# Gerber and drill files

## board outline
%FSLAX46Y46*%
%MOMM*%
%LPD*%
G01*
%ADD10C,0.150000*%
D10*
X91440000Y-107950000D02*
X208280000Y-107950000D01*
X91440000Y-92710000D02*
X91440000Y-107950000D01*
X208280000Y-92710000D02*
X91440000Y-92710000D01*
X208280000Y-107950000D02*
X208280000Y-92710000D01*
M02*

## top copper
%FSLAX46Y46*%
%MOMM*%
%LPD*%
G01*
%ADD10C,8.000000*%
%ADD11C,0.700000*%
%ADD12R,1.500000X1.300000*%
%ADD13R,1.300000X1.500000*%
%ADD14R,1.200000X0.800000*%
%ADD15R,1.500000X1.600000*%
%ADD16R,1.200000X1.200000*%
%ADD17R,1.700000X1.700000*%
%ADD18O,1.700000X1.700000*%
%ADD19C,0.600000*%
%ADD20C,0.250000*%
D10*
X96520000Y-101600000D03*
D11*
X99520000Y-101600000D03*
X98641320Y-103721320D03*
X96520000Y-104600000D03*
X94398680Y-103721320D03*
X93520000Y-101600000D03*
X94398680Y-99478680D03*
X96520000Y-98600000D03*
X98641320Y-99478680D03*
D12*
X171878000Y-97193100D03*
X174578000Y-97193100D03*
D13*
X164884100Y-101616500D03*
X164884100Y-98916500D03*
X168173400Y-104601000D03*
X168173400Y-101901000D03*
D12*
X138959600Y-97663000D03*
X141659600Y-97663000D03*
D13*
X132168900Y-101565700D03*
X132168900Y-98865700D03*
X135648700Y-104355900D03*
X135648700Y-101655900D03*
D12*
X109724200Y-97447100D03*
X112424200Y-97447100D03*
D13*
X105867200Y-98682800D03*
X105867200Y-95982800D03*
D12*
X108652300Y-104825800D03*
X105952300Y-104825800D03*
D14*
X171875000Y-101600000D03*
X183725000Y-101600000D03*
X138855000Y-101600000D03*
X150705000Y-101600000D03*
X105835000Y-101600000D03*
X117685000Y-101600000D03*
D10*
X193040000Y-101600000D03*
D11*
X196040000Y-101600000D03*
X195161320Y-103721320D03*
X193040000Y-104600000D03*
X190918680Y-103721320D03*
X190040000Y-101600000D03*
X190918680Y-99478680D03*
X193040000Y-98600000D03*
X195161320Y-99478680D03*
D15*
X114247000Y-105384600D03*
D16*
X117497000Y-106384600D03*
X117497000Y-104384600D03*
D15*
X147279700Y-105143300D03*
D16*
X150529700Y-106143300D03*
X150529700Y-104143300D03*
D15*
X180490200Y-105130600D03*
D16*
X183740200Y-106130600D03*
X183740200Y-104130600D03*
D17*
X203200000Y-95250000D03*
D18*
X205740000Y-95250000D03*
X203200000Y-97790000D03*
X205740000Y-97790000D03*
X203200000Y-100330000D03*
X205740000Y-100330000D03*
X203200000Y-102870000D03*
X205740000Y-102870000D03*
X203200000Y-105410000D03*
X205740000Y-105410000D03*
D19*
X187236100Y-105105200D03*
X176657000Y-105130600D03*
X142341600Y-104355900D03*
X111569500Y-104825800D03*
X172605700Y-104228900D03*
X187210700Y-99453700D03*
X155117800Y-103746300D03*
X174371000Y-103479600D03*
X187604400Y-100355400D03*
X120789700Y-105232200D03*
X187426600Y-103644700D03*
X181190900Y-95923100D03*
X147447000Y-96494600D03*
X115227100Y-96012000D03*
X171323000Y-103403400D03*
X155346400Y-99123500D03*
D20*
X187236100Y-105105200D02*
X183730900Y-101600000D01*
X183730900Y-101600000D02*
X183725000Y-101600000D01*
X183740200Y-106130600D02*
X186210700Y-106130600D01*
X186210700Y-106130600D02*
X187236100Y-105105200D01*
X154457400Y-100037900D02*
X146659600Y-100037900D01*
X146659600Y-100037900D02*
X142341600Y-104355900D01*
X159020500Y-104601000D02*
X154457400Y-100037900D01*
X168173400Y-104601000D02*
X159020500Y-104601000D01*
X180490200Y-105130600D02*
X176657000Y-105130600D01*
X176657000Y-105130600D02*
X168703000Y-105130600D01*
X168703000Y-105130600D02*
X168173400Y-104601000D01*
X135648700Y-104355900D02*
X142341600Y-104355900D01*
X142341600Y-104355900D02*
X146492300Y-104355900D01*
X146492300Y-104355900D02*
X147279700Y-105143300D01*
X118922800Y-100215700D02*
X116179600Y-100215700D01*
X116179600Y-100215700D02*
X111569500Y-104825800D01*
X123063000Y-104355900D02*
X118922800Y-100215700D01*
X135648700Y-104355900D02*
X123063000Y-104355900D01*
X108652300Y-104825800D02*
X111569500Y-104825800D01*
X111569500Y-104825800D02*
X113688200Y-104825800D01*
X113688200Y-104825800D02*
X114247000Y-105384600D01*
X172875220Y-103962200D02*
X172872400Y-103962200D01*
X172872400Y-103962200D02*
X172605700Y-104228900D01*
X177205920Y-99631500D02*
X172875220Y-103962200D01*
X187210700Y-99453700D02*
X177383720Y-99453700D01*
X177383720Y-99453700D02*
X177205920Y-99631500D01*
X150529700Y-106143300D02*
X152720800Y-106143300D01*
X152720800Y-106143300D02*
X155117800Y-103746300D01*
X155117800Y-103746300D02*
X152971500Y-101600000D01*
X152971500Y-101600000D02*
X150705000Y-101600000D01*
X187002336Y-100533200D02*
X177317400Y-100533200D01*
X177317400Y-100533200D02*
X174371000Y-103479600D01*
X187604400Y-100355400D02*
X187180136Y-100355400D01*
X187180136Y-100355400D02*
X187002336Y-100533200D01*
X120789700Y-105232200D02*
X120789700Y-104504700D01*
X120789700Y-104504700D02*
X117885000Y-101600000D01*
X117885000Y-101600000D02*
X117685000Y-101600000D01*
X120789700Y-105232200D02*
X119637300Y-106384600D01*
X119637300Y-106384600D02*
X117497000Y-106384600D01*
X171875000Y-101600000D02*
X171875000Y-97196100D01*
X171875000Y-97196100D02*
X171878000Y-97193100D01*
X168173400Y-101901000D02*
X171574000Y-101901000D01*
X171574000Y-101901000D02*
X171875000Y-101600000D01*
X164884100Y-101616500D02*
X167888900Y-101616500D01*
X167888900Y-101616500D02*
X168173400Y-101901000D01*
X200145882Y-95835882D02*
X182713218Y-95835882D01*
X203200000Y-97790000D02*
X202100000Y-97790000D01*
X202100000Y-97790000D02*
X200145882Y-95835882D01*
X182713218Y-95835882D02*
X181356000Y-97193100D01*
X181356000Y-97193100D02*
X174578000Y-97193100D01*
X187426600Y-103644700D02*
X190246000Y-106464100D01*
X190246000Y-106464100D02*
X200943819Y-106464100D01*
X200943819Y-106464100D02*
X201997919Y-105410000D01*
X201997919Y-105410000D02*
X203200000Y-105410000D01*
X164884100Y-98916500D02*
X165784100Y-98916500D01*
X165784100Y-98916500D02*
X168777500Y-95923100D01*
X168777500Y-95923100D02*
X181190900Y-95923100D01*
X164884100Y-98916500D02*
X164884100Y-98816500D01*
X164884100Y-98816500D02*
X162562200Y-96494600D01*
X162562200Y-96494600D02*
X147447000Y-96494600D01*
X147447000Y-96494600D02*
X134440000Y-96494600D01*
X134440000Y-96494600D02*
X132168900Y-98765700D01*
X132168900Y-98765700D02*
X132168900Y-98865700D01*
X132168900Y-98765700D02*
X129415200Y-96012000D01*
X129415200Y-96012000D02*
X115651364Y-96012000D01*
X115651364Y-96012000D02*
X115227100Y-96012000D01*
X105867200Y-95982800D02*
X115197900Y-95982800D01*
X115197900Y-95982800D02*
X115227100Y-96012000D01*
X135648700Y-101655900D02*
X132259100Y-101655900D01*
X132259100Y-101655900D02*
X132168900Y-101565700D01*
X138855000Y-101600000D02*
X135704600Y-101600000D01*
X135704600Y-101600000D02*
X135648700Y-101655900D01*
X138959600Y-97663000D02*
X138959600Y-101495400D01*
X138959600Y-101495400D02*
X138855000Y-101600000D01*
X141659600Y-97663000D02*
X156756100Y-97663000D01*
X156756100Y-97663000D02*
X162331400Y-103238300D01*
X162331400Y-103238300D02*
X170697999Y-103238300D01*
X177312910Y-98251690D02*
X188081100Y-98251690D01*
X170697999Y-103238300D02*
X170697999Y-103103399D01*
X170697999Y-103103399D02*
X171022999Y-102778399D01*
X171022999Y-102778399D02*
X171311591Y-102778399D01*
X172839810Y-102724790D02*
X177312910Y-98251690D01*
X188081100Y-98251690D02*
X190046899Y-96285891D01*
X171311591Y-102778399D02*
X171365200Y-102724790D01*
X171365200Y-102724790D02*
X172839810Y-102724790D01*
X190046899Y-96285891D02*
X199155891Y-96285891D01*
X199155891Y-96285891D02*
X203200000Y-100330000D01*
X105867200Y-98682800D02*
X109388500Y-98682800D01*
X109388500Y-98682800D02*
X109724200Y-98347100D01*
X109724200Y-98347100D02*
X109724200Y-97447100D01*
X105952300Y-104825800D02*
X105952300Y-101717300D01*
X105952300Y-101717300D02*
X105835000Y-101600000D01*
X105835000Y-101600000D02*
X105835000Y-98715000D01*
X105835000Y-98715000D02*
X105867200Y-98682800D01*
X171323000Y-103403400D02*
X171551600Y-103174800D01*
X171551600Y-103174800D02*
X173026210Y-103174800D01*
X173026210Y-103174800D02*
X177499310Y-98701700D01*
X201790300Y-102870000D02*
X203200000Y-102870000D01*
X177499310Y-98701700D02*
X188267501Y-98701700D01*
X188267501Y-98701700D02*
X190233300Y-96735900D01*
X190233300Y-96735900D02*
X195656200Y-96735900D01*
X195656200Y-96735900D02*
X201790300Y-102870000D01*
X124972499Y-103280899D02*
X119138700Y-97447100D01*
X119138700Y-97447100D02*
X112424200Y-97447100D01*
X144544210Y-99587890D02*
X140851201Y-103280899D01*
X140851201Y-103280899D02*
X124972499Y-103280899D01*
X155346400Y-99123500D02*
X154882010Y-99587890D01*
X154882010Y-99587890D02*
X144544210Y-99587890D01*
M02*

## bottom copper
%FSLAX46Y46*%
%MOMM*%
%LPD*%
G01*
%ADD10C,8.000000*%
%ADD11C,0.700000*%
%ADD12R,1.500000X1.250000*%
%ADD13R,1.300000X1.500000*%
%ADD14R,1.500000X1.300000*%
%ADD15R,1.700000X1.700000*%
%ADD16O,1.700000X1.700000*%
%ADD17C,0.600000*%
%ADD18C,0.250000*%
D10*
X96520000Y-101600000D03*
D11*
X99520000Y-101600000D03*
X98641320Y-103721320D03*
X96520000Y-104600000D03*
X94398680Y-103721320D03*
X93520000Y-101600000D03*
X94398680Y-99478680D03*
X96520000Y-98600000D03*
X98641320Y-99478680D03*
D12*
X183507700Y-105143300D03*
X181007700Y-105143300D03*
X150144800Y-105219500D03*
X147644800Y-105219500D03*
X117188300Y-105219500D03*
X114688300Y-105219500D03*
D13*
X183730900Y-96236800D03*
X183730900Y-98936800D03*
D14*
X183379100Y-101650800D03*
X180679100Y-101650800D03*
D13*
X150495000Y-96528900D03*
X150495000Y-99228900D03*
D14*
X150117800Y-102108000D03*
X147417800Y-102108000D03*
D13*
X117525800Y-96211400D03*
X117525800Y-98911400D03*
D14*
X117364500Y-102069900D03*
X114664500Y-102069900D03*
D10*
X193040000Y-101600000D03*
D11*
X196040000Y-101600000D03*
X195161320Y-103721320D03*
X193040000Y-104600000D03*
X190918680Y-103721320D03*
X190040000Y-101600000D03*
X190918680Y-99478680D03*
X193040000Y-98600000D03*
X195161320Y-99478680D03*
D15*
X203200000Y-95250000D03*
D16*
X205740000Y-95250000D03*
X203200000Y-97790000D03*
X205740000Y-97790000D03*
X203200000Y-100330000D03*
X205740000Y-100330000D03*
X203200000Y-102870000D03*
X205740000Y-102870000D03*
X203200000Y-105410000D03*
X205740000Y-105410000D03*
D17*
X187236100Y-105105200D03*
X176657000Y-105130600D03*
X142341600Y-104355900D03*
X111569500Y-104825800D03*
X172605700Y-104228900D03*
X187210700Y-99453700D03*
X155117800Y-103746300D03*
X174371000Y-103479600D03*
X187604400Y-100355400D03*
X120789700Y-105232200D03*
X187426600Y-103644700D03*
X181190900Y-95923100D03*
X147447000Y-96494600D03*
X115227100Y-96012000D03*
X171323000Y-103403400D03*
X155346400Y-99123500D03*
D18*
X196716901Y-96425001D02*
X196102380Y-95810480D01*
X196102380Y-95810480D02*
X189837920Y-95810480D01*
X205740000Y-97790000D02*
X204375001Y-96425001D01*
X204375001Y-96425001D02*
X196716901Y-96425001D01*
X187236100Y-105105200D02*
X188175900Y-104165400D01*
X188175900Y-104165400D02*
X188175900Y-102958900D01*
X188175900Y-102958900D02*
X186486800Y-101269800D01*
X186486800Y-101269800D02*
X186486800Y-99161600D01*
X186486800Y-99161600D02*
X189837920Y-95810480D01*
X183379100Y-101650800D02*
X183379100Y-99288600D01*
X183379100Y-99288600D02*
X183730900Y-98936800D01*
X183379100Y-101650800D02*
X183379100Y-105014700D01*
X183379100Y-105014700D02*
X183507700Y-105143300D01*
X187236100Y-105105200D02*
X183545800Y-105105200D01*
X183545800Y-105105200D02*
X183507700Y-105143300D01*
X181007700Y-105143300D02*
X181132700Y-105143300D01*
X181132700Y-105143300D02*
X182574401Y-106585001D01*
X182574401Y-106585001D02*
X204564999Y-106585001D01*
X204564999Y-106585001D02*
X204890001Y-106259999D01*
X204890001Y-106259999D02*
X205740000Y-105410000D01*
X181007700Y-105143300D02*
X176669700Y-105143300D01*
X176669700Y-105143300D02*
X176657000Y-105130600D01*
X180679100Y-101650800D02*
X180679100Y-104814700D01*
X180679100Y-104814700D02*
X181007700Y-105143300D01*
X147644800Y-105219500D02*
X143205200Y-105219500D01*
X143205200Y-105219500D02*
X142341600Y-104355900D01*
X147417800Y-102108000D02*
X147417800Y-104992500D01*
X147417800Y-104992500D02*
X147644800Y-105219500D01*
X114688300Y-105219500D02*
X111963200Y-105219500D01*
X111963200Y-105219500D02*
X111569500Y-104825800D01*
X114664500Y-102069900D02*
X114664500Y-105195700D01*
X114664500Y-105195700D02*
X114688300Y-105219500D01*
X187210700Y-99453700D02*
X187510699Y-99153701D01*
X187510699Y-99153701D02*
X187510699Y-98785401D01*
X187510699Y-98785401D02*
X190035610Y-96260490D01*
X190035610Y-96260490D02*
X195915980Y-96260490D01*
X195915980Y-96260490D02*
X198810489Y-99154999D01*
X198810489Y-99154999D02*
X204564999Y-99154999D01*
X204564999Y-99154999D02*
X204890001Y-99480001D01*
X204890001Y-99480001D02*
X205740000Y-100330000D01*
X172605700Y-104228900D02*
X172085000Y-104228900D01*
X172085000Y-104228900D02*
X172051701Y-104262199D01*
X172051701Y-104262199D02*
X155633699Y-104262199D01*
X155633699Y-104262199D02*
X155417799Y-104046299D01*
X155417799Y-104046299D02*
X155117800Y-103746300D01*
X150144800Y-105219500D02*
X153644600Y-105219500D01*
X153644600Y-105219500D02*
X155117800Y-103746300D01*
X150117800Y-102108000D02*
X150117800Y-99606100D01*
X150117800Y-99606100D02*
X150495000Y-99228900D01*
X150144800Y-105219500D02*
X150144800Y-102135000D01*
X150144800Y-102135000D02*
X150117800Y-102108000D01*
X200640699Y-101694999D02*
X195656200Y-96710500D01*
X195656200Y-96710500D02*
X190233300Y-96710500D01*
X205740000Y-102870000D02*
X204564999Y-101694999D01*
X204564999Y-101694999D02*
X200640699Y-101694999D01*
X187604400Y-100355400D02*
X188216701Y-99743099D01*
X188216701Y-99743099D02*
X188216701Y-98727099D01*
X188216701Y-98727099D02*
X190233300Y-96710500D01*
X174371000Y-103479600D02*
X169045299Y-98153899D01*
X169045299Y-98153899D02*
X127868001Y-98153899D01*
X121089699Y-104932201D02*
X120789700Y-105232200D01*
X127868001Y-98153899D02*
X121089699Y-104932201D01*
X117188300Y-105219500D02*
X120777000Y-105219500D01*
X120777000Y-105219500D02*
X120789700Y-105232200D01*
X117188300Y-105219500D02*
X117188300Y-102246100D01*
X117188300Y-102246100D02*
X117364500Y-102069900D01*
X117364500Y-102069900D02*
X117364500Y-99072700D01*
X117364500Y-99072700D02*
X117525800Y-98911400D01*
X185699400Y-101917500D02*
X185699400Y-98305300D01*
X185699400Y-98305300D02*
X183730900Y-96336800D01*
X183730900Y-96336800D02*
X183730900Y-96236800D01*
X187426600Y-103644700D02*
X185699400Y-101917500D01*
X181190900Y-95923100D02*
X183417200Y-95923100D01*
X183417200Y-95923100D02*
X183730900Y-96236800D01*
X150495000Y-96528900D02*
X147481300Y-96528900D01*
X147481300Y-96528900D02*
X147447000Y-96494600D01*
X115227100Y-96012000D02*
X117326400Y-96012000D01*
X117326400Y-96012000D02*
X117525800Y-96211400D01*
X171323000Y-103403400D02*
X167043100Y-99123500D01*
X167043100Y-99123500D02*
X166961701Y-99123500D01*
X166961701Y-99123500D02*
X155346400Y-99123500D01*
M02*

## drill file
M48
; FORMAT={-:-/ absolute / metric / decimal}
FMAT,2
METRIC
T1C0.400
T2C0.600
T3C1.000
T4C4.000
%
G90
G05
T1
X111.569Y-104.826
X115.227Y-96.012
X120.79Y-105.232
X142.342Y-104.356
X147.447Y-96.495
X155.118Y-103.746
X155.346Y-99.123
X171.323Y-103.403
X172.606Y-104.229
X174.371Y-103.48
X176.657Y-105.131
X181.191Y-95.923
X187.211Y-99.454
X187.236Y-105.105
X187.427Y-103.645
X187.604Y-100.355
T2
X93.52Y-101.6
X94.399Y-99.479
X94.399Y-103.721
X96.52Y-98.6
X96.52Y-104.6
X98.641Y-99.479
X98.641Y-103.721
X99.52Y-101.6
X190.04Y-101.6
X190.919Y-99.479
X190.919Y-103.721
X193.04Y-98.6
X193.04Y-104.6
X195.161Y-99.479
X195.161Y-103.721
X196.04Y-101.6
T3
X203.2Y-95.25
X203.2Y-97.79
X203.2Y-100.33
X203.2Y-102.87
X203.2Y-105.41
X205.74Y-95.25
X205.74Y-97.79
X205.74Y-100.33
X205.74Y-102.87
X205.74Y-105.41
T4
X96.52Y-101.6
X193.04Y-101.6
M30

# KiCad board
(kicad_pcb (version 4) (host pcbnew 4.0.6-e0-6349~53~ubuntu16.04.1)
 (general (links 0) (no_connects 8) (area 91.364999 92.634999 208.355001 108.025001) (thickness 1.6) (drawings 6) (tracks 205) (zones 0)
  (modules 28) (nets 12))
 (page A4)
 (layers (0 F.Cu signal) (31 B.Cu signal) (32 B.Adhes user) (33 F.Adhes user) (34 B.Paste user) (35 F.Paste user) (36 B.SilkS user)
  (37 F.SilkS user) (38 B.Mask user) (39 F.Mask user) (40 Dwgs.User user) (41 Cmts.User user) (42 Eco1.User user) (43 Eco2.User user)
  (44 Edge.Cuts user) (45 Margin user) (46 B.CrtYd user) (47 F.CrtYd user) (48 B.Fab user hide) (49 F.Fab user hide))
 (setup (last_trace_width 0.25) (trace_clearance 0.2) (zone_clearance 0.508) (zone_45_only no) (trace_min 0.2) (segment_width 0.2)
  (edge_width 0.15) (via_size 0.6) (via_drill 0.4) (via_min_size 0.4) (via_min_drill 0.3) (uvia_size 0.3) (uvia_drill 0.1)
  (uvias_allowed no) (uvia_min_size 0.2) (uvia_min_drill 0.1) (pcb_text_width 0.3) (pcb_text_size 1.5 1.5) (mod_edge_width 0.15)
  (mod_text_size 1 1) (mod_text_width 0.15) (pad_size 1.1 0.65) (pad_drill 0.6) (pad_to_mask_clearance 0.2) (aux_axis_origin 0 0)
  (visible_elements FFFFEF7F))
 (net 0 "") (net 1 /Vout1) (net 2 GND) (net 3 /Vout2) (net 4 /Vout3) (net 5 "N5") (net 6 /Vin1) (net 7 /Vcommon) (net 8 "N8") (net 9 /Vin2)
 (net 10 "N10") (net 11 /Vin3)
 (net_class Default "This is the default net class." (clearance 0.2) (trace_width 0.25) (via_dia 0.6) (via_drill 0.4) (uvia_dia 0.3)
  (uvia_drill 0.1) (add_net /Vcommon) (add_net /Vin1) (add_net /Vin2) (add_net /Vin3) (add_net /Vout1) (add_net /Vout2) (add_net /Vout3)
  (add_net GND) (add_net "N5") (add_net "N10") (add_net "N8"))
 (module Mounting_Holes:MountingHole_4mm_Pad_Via (layer F.Cu) (at 96.52 101.6)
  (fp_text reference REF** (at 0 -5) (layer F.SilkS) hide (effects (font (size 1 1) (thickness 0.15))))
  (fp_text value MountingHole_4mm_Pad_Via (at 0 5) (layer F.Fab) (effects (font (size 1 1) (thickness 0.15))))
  (pad 1 thru_hole circle (at 0 0) (size 8 8) (drill 4) (layers *.Cu *.Mask))
  (pad "" thru_hole circle (at 3 0) (size 0.7 0.7) (drill 0.6) (layers *.Cu *.Mask))
  (pad "" thru_hole circle (at 2.12132 2.12132) (size 0.7 0.7) (drill 0.6) (layers *.Cu *.Mask))
  (pad "" thru_hole circle (at 0 3) (size 0.7 0.7) (drill 0.6) (layers *.Cu *.Mask))
  (pad "" thru_hole circle (at -2.12132 2.12132) (size 0.7 0.7) (drill 0.6) (layers *.Cu *.Mask))
  (pad "" thru_hole circle (at -3 0) (size 0.7 0.7) (drill 0.6) (layers *.Cu *.Mask))
  (pad "" thru_hole circle (at -2.12132 -2.12132) (size 0.7 0.7) (drill 0.6) (layers *.Cu *.Mask))
  (pad "" thru_hole circle (at 0 -3) (size 0.7 0.7) (drill 0.6) (layers *.Cu *.Mask))
  (pad "" thru_hole circle (at 2.12132 -2.12132) (size 0.7 0.7) (drill 0.6) (layers *.Cu *.Mask)))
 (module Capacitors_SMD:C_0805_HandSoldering (layer B.Cu) (at 182.2577 105.1433 180)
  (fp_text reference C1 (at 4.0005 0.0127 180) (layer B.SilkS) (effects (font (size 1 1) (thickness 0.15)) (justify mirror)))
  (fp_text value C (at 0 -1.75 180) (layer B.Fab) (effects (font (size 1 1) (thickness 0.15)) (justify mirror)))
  (pad 1 smd rect (at -1.25 0 180) (size 1.5 1.25) (layers B.Cu B.Paste B.Mask) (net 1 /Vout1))
  (pad 2 smd rect (at 1.25 0 180) (size 1.5 1.25) (layers B.Cu B.Paste B.Mask) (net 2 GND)))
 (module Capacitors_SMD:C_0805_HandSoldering (layer B.Cu) (at 148.8948 105.2195 180)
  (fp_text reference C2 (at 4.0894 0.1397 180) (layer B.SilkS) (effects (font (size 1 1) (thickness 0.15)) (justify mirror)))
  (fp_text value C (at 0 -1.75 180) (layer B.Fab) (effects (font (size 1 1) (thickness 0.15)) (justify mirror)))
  (pad 1 smd rect (at -1.25 0 180) (size 1.5 1.25) (layers B.Cu B.Paste B.Mask) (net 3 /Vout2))
  (pad 2 smd rect (at 1.25 0 180) (size 1.5 1.25) (layers B.Cu B.Paste B.Mask) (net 2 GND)))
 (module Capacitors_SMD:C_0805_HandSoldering (layer B.Cu) (at 115.9383 105.2195 180)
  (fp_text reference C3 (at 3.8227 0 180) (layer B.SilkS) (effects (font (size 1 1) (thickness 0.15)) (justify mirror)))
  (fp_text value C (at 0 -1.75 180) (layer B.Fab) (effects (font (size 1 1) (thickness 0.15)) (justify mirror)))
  (pad 1 smd rect (at -1.25 0 180) (size 1.5 1.25) (layers B.Cu B.Paste B.Mask) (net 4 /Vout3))
  (pad 2 smd rect (at 1.25 0 180) (size 1.5 1.25) (layers B.Cu B.Paste B.Mask) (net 2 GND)))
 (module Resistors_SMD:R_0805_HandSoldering (layer F.Cu) (at 173.228 97.1931)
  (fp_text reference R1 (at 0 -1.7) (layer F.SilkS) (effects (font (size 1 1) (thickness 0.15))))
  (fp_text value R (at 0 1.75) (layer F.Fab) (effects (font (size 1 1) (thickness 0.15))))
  (pad 1 smd rect (at -1.35 0) (size 1.5 1.3) (layers F.Cu F.Paste F.Mask) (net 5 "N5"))
  (pad 2 smd rect (at 1.35 0) (size 1.5 1.3) (layers F.Cu F.Paste F.Mask) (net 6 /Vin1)))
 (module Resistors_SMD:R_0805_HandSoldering (layer F.Cu) (at 164.8841 100.2665 90)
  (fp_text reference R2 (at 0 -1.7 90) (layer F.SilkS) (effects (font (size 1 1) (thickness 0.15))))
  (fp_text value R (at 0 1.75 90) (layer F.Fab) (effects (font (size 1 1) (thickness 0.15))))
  (pad 1 smd rect (at -1.35 0 90) (size 1.5 1.3) (layers F.Cu F.Paste F.Mask) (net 5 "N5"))
  (pad 2 smd rect (at 1.35 0 90) (size 1.5 1.3) (layers F.Cu F.Paste F.Mask) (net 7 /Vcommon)))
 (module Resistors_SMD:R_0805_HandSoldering (layer F.Cu) (at 168.1734 103.251 90)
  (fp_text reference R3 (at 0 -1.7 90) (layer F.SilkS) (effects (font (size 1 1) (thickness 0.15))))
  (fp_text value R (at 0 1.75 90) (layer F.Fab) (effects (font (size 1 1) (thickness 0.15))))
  (pad 1 smd rect (at -1.35 0 90) (size 1.5 1.3) (layers F.Cu F.Paste F.Mask) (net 2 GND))
  (pad 2 smd rect (at 1.35 0 90) (size 1.5 1.3) (layers F.Cu F.Paste F.Mask) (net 5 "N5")))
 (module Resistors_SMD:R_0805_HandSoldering (layer B.Cu) (at 183.7309 97.5868 270)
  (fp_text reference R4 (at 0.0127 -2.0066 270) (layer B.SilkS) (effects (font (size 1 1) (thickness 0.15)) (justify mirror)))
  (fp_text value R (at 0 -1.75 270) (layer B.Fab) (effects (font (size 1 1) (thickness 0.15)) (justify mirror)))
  (pad 1 smd rect (at -1.35 0 270) (size 1.5 1.3) (layers B.Cu B.Paste B.Mask) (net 7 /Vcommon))
  (pad 2 smd rect (at 1.35 0 270) (size 1.5 1.3) (layers B.Cu B.Paste B.Mask) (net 1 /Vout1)))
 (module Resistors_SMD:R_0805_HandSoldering (layer B.Cu) (at 182.0291 101.6508 180)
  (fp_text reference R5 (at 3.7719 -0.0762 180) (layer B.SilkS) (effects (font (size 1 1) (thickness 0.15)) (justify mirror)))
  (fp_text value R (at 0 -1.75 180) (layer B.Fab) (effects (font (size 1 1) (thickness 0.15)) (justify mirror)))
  (pad 1 smd rect (at -1.35 0 180) (size 1.5 1.3) (layers B.Cu B.Paste B.Mask) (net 1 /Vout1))
  (pad 2 smd rect (at 1.35 0 180) (size 1.5 1.3) (layers B.Cu B.Paste B.Mask) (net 2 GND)))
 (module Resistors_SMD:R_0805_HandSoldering (layer F.Cu) (at 140.3096 97.663)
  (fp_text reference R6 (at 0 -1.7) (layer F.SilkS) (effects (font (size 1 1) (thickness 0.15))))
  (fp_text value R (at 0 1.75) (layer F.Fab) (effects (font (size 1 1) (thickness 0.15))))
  (pad 1 smd rect (at -1.35 0) (size 1.5 1.3) (layers F.Cu F.Paste F.Mask) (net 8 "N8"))
  (pad 2 smd rect (at 1.35 0) (size 1.5 1.3) (layers F.Cu F.Paste F.Mask) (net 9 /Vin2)))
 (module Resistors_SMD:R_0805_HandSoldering (layer F.Cu) (at 132.1689 100.2157 90)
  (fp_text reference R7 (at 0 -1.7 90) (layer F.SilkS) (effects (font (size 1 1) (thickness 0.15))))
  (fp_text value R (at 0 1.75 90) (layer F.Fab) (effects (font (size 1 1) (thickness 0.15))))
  (pad 1 smd rect (at -1.35 0 90) (size 1.5 1.3) (layers F.Cu F.Paste F.Mask) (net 8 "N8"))
  (pad 2 smd rect (at 1.35 0 90) (size 1.5 1.3) (layers F.Cu F.Paste F.Mask) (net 7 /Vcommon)))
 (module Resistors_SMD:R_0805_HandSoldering (layer F.Cu) (at 135.6487 103.0059 90)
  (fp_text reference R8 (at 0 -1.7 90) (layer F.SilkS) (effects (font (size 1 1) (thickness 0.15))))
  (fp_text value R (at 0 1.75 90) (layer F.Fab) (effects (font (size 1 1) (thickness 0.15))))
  (pad 1 smd rect (at -1.35 0 90) (size 1.5 1.3) (layers F.Cu F.Paste F.Mask) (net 2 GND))
  (pad 2 smd rect (at 1.35 0 90) (size 1.5 1.3) (layers F.Cu F.Paste F.Mask) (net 8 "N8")))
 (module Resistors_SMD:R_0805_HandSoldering (layer B.Cu) (at 150.495 97.8789 270)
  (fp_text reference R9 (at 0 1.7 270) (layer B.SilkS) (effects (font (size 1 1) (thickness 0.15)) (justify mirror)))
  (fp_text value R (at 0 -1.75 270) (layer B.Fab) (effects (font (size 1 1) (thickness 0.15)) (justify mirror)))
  (pad 1 smd rect (at -1.35 0 270) (size 1.5 1.3) (layers B.Cu B.Paste B.Mask) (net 7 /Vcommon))
  (pad 2 smd rect (at 1.35 0 270) (size 1.5 1.3) (layers B.Cu B.Paste B.Mask) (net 3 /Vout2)))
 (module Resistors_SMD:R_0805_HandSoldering (layer B.Cu) (at 148.7678 102.108 180)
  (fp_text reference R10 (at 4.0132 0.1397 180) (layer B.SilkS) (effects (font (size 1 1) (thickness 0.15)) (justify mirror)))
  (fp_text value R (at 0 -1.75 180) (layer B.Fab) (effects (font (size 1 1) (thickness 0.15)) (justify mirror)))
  (pad 1 smd rect (at -1.35 0 180) (size 1.5 1.3) (layers B.Cu B.Paste B.Mask) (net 3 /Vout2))
  (pad 2 smd rect (at 1.35 0 180) (size 1.5 1.3) (layers B.Cu B.Paste B.Mask) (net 2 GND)))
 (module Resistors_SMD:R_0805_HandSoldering (layer F.Cu) (at 111.0742 97.4471)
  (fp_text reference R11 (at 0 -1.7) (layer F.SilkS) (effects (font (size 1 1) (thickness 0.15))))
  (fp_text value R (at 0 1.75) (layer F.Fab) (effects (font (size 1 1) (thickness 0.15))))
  (pad 1 smd rect (at -1.35 0) (size 1.5 1.3) (layers F.Cu F.Paste F.Mask) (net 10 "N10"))
  (pad 2 smd rect (at 1.35 0) (size 1.5 1.3) (layers F.Cu F.Paste F.Mask) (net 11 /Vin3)))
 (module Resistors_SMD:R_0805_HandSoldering (layer F.Cu) (at 105.8672 97.3328 90)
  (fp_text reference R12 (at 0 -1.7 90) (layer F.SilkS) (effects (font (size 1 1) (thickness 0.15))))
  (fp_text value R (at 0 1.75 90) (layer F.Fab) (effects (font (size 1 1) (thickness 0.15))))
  (pad 1 smd rect (at -1.35 0 90) (size 1.5 1.3) (layers F.Cu F.Paste F.Mask) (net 10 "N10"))
  (pad 2 smd rect (at 1.35 0 90) (size 1.5 1.3) (layers F.Cu F.Paste F.Mask) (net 7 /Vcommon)))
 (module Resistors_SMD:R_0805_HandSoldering (layer F.Cu) (at 107.3023 104.8258 180)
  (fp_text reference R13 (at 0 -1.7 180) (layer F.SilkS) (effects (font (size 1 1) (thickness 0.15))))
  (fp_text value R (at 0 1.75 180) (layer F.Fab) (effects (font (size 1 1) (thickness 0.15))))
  (pad 1 smd rect (at -1.35 0 180) (size 1.5 1.3) (layers F.Cu F.Paste F.Mask) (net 2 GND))
  (pad 2 smd rect (at 1.35 0 180) (size 1.5 1.3) (layers F.Cu F.Paste F.Mask) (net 10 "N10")))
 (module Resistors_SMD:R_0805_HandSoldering (layer B.Cu) (at 117.5258 97.5614 270)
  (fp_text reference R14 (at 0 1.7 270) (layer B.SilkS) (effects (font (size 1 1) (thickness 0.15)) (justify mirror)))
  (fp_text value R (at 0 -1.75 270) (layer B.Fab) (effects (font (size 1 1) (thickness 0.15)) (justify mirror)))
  (pad 1 smd rect (at -1.35 0 270) (size 1.5 1.3) (layers B.Cu B.Paste B.Mask) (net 7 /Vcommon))
  (pad 2 smd rect (at 1.35 0 270) (size 1.5 1.3) (layers B.Cu B.Paste B.Mask) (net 4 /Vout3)))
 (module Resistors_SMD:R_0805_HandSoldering (layer B.Cu) (at 116.0145 102.0699 180)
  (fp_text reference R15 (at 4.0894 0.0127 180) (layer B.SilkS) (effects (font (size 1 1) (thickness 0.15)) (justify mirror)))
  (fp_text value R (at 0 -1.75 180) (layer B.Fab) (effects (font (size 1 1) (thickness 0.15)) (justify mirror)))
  (pad 1 smd rect (at -1.35 0 180) (size 1.5 1.3) (layers B.Cu B.Paste B.Mask) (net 4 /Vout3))
  (pad 2 smd rect (at 1.35 0 180) (size 1.5 1.3) (layers B.Cu B.Paste B.Mask) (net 2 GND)))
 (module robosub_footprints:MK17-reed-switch (layer F.Cu) (at 177.8 101.6)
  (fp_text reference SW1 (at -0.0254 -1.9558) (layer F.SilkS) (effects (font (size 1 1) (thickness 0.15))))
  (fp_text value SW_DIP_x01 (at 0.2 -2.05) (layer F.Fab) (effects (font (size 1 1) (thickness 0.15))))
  (pad 1 smd rect (at -5.925 0) (size 1.2 0.8) (layers F.Cu F.Paste F.Mask) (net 5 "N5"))
  (pad 2 smd rect (at 5.925 0) (size 1.2 0.8) (layers F.Cu F.Paste F.Mask) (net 1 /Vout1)))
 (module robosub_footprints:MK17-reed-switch (layer F.Cu) (at 144.78 101.6)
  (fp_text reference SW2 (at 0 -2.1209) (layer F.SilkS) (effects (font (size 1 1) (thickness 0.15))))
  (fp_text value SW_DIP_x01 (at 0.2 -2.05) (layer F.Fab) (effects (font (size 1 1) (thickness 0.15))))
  (pad 1 smd rect (at -5.925 0) (size 1.2 0.8) (layers F.Cu F.Paste F.Mask) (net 8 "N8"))
  (pad 2 smd rect (at 5.925 0) (size 1.2 0.8) (layers F.Cu F.Paste F.Mask) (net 3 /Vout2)))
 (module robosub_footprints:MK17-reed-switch (layer F.Cu) (at 111.76 101.6)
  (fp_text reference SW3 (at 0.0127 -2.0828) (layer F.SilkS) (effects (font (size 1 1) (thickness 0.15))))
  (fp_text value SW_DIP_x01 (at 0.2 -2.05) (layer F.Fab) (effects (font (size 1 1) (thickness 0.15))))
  (pad 1 smd rect (at -5.925 0) (size 1.2 0.8) (layers F.Cu F.Paste F.Mask) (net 10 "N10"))
  (pad 2 smd rect (at 5.925 0) (size 1.2 0.8) (layers F.Cu F.Paste F.Mask) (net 4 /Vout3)))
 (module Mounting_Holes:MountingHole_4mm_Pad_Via (layer F.Cu) (at 193.04 101.6)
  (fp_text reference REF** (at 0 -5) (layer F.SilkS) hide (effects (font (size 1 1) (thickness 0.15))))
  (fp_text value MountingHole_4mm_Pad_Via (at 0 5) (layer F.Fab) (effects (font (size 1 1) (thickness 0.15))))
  (pad 1 thru_hole circle (at 0 0) (size 8 8) (drill 4) (layers *.Cu *.Mask))
  (pad "" thru_hole circle (at 3 0) (size 0.7 0.7) (drill 0.6) (layers *.Cu *.Mask))
  (pad "" thru_hole circle (at 2.12132 2.12132) (size 0.7 0.7) (drill 0.6) (layers *.Cu *.Mask))
  (pad "" thru_hole circle (at 0 3) (size 0.7 0.7) (drill 0.6) (layers *.Cu *.Mask))
  (pad "" thru_hole circle (at -2.12132 2.12132) (size 0.7 0.7) (drill 0.6) (layers *.Cu *.Mask))
  (pad "" thru_hole circle (at -3 0) (size 0.7 0.7) (drill 0.6) (layers *.Cu *.Mask))
  (pad "" thru_hole circle (at -2.12132 -2.12132) (size 0.7 0.7) (drill 0.6) (layers *.Cu *.Mask))
  (pad "" thru_hole circle (at 0 -3) (size 0.7 0.7) (drill 0.6) (layers *.Cu *.Mask))
  (pad "" thru_hole circle (at 2.12132 -2.12132) (size 0.7 0.7) (drill 0.6) (layers *.Cu *.Mask)))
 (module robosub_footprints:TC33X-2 (layer F.Cu) (at 115.697 105.3846 90)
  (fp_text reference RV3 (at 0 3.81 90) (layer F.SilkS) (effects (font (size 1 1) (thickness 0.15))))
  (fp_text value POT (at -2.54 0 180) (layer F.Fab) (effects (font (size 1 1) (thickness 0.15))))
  (pad 2 smd rect (at 0 -1.45 90) (size 1.6 1.5) (layers F.Cu F.Paste F.Mask) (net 2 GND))
  (pad 1 smd rect (at -1 1.8 90) (size 1.2 1.2) (layers F.Cu F.Paste F.Mask) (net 4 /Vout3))
  (pad 3 smd rect (at 1 1.8 90) (size 1.2 1.2) (layers F.Cu F.Paste F.Mask)))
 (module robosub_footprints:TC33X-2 (layer F.Cu) (at 148.7297 105.1433 90)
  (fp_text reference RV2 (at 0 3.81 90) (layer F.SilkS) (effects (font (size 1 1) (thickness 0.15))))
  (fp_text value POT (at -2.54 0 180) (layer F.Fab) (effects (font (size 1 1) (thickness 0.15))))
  (pad 2 smd rect (at 0 -1.45 90) (size 1.6 1.5) (layers F.Cu F.Paste F.Mask) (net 2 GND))
  (pad 1 smd rect (at -1 1.8 90) (size 1.2 1.2) (layers F.Cu F.Paste F.Mask) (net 3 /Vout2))
  (pad 3 smd rect (at 1 1.8 90) (size 1.2 1.2) (layers F.Cu F.Paste F.Mask)))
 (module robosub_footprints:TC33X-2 (layer F.Cu) (at 181.9402 105.1306 90)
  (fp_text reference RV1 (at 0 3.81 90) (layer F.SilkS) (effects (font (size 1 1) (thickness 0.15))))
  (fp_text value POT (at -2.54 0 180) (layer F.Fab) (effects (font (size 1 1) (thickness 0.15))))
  (pad 2 smd rect (at 0 -1.45 90) (size 1.6 1.5) (layers F.Cu F.Paste F.Mask) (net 2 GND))
  (pad 1 smd rect (at -1 1.8 90) (size 1.2 1.2) (layers F.Cu F.Paste F.Mask) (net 1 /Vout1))
  (pad 3 smd rect (at 1 1.8 90) (size 1.2 1.2) (layers F.Cu F.Paste F.Mask)))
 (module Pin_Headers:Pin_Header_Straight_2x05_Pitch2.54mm (layer F.Cu) (at 203.2 95.25)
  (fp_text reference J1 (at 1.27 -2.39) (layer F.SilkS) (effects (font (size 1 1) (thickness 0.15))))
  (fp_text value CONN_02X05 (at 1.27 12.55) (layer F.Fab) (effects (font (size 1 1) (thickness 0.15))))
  (pad 1 thru_hole rect (at 0 0) (size 1.7 1.7) (drill 1) (layers *.Cu *.Mask))
  (pad 2 thru_hole oval (at 2.54 0) (size 1.7 1.7) (drill 1) (layers *.Cu *.Mask))
  (pad 3 thru_hole oval (at 0 2.54) (size 1.7 1.7) (drill 1) (layers *.Cu *.Mask) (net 6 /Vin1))
  (pad 4 thru_hole oval (at 2.54 2.54) (size 1.7 1.7) (drill 1) (layers *.Cu *.Mask) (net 1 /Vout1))
  (pad 5 thru_hole oval (at 0 5.08) (size 1.7 1.7) (drill 1) (layers *.Cu *.Mask) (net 9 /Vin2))
  (pad 6 thru_hole oval (at 2.54 5.08) (size 1.7 1.7) (drill 1) (layers *.Cu *.Mask) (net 3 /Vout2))
  (pad 7 thru_hole oval (at 0 7.62) (size 1.7 1.7) (drill 1) (layers *.Cu *.Mask) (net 11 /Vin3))
  (pad 8 thru_hole oval (at 2.54 7.62) (size 1.7 1.7) (drill 1) (layers *.Cu *.Mask) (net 4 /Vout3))
  (pad 9 thru_hole oval (at 0 10.16) (size 1.7 1.7) (drill 1) (layers *.Cu *.Mask) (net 7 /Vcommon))
  (pad 10 thru_hole oval (at 2.54 10.16) (size 1.7 1.7) (drill 1) (layers *.Cu *.Mask) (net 2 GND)))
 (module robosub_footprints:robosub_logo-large (layer B.Cu) (at 167.64 98.7806 180)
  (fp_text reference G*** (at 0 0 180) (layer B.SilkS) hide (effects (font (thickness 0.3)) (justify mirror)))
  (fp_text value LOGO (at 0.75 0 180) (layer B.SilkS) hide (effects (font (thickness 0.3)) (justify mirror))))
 (gr_line (start 91.44 107.95) (end 208.28 107.95) (layer Edge.Cuts) (width 0.15))
 (gr_line (start 91.44 92.71) (end 91.44 107.95) (layer Edge.Cuts) (width 0.15))
 (gr_line (start 208.28 92.71) (end 91.44 92.71) (layer Edge.Cuts) (width 0.15))
 (gr_line (start 208.28 107.95) (end 208.28 92.71) (layer Edge.Cuts) (width 0.15))
 (segment (start 196.716901 96.425001) (end 196.10238 95.81048) (width 0.25) (layer B.Cu) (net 1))
 (segment (start 196.10238 95.81048) (end 189.83792 95.81048) (width 0.25) (layer B.Cu) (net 1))
 (segment (start 205.74 97.79) (end 204.375001 96.425001) (width 0.25) (layer B.Cu) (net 1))
 (segment (start 204.375001 96.425001) (end 196.716901 96.425001) (width 0.25) (layer B.Cu) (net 1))
 (segment (start 187.2361 105.1052) (end 188.1759 104.1654) (width 0.25) (layer B.Cu) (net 1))
 (segment (start 188.1759 104.1654) (end 188.1759 102.9589) (width 0.25) (layer B.Cu) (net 1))
 (segment (start 188.1759 102.9589) (end 186.4868 101.2698) (width 0.25) (layer B.Cu) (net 1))
 (segment (start 186.4868 101.2698) (end 186.4868 99.1616) (width 0.25) (layer B.Cu) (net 1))
 (segment (start 186.4868 99.1616) (end 189.83792 95.81048) (width 0.25) (layer B.Cu) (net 1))
 (segment (start 187.2361 105.1052) (end 183.7309 101.6) (width 0.25) (layer F.Cu) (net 1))
 (segment (start 183.7309 101.6) (end 183.725 101.6) (width 0.25) (layer F.Cu) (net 1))
 (segment (start 183.3791 101.6508) (end 183.3791 99.2886) (width 0.25) (layer B.Cu) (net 1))
 (segment (start 183.3791 99.2886) (end 183.7309 98.9368) (width 0.25) (layer B.Cu) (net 1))
 (segment (start 183.3791 101.6508) (end 183.3791 105.0147) (width 0.25) (layer B.Cu) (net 1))
 (segment (start 183.3791 105.0147) (end 183.5077 105.1433) (width 0.25) (layer B.Cu) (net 1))
 (segment (start 187.2361 105.1052) (end 183.5458 105.1052) (width 0.25) (layer B.Cu) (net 1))
 (segment (start 183.5458 105.1052) (end 183.5077 105.1433) (width 0.25) (layer B.Cu) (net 1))
 (segment (start 183.7402 106.1306) (end 186.2107 106.1306) (width 0.25) (layer F.Cu) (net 1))
 (via (at 187.2361 105.1052) (size 0.6) (drill 0.4) (layers F.Cu B.Cu) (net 1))
 (segment (start 186.2107 106.1306) (end 187.2361 105.1052) (width 0.25) (layer F.Cu) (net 1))
 (segment (start 181.0077 105.1433) (end 181.1327 105.1433) (width 0.25) (layer B.Cu) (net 2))
 (segment (start 181.1327 105.1433) (end 182.574401 106.585001) (width 0.25) (layer B.Cu) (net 2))
 (segment (start 182.574401 106.585001) (end 204.564999 106.585001) (width 0.25) (layer B.Cu) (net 2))
 (segment (start 204.564999 106.585001) (end 204.890001 106.259999) (width 0.25) (layer B.Cu) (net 2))
 (segment (start 204.890001 106.259999) (end 205.74 105.41) (width 0.25) (layer B.Cu) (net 2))
 (segment (start 154.4574 100.0379) (end 146.6596 100.0379) (width 0.25) (layer F.Cu) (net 2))
 (segment (start 146.6596 100.0379) (end 142.3416 104.3559) (width 0.25) (layer F.Cu) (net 2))
 (segment (start 159.0205 104.601) (end 154.4574 100.0379) (width 0.25) (layer F.Cu) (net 2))
 (segment (start 168.1734 104.601) (end 159.0205 104.601) (width 0.25) (layer F.Cu) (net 2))
 (segment (start 180.4902 105.1306) (end 176.657 105.1306) (width 0.25) (layer F.Cu) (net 2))
 (segment (start 176.657 105.1306) (end 168.703 105.1306) (width 0.25) (layer F.Cu) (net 2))
 (segment (start 181.0077 105.1433) (end 176.6697 105.1433) (width 0.25) (layer B.Cu) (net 2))
 (segment (start 176.6697 105.1433) (end 176.657 105.1306) (width 0.25) (layer B.Cu) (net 2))
 (via (at 176.657 105.1306) (size 0.6) (drill 0.4) (layers F.Cu B.Cu) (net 2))
 (segment (start 180.6791 101.6508) (end 180.6791 104.8147) (width 0.25) (layer B.Cu) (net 2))
 (segment (start 180.6791 104.8147) (end 181.0077 105.1433) (width 0.25) (layer B.Cu) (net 2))
 (segment (start 168.703 105.1306) (end 168.1734 104.601) (width 0.25) (layer F.Cu) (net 2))
 (segment (start 135.6487 104.3559) (end 142.3416 104.3559) (width 0.25) (layer F.Cu) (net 2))
 (segment (start 142.3416 104.3559) (end 146.4923 104.3559) (width 0.25) (layer F.Cu) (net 2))
 (segment (start 147.6448 105.2195) (end 143.2052 105.2195) (width 0.25) (layer B.Cu) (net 2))
 (segment (start 143.2052 105.2195) (end 142.3416 104.3559) (width 0.25) (layer B.Cu) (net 2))
 (via (at 142.3416 104.3559) (size 0.6) (drill 0.4) (layers F.Cu B.Cu) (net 2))
 (segment (start 147.4178 102.108) (end 147.4178 104.9925) (width 0.25) (layer B.Cu) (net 2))
 (segment (start 147.4178 104.9925) (end 147.6448 105.2195) (width 0.25) (layer B.Cu) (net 2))
 (segment (start 146.4923 104.3559) (end 147.2797 105.1433) (width 0.25) (layer F.Cu) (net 2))
 (segment (start 118.9228 100.2157) (end 116.1796 100.2157) (width 0.25) (layer F.Cu) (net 2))
 (segment (start 116.1796 100.2157) (end 111.5695 104.8258) (width 0.25) (layer F.Cu) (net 2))
 (segment (start 123.063 104.3559) (end 118.9228 100.2157) (width 0.25) (layer F.Cu) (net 2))
 (segment (start 135.6487 104.3559) (end 123.063 104.3559) (width 0.25) (layer F.Cu) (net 2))
 (segment (start 108.6523 104.8258) (end 111.5695 104.8258) (width 0.25) (layer F.Cu) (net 2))
 (segment (start 111.5695 104.8258) (end 113.6882 104.8258) (width 0.25) (layer F.Cu) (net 2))
 (segment (start 114.6883 105.2195) (end 111.9632 105.2195) (width 0.25) (layer B.Cu) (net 2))
 (segment (start 111.9632 105.2195) (end 111.5695 104.8258) (width 0.25) (layer B.Cu) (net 2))
 (via (at 111.5695 104.8258) (size 0.6) (drill 0.4) (layers F.Cu B.Cu) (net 2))
 (segment (start 114.6645 102.0699) (end 114.6645 105.1957) (width 0.25) (layer B.Cu) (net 2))
 (segment (start 114.6645 105.1957) (end 114.6883 105.2195) (width 0.25) (layer B.Cu) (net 2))
 (segment (start 113.6882 104.8258) (end 114.247 105.3846) (width 0.25) (layer F.Cu) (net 2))
 (segment (start 187.2107 99.4537) (end 187.510699 99.153701) (width 0.25) (layer B.Cu) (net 3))
 (segment (start 187.510699 99.153701) (end 187.510699 98.785401) (width 0.25) (layer B.Cu) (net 3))
 (segment (start 187.510699 98.785401) (end 190.03561 96.26049) (width 0.25) (layer B.Cu) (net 3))
 (segment (start 190.03561 96.26049) (end 195.91598 96.26049) (width 0.25) (layer B.Cu) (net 3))
 (segment (start 195.91598 96.26049) (end 198.810489 99.154999) (width 0.25) (layer B.Cu) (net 3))
 (segment (start 198.810489 99.154999) (end 204.564999 99.154999) (width 0.25) (layer B.Cu) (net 3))
 (segment (start 204.564999 99.154999) (end 204.890001 99.480001) (width 0.25) (layer B.Cu) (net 3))
 (segment (start 204.890001 99.480001) (end 205.74 100.33) (width 0.25) (layer B.Cu) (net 3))
 (segment (start 172.6057 104.2289) (end 172.085 104.2289) (width 0.25) (layer B.Cu) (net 3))
 (segment (start 172.085 104.2289) (end 172.051701 104.262199) (width 0.25) (layer B.Cu) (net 3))
 (segment (start 172.87522 103.9622) (end 172.8724 103.9622) (width 0.25) (layer F.Cu) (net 3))
 (segment (start 172.8724 103.9622) (end 172.6057 104.2289) (width 0.25) (layer F.Cu) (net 3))
 (via (at 172.6057 104.2289) (size 0.6) (drill 0.4) (layers F.Cu B.Cu) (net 3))
 (segment (start 177.20592 99.6315) (end 172.87522 103.9622) (width 0.25) (layer F.Cu) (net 3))
 (segment (start 187.2107 99.4537) (end 177.38372 99.4537) (width 0.25) (layer F.Cu) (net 3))
 (segment (start 177.38372 99.4537) (end 177.20592 99.6315) (width 0.25) (layer F.Cu) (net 3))
 (via (at 187.2107 99.4537) (size 0.6) (drill 0.4) (layers F.Cu B.Cu) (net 3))
 (segment (start 172.051701 104.262199) (end 155.633699 104.262199) (width 0.25) (layer B.Cu) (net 3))
 (segment (start 155.633699 104.262199) (end 155.417799 104.046299) (width 0.25) (layer B.Cu) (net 3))
 (segment (start 155.417799 104.046299) (end 155.1178 103.7463) (width 0.25) (layer B.Cu) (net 3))
 (segment (start 150.5297 106.1433) (end 152.7208 106.1433) (width 0.25) (layer F.Cu) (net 3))
 (segment (start 152.7208 106.1433) (end 155.1178 103.7463) (width 0.25) (layer F.Cu) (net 3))
 (segment (start 155.1178 103.7463) (end 152.9715 101.6) (width 0.25) (layer F.Cu) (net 3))
 (segment (start 152.9715 101.6) (end 150.705 101.6) (width 0.25) (layer F.Cu) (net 3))
 (segment (start 150.1448 105.2195) (end 153.6446 105.2195) (width 0.25) (layer B.Cu) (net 3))
 (segment (start 153.6446 105.2195) (end 155.1178 103.7463) (width 0.25) (layer B.Cu) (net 3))
 (via (at 155.1178 103.7463) (size 0.6) (drill 0.4) (layers F.Cu B.Cu) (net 3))
 (segment (start 150.1178 102.108) (end 150.1178 99.6061) (width 0.25) (layer B.Cu) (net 3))
 (segment (start 150.1178 99.6061) (end 150.495 99.2289) (width 0.25) (layer B.Cu) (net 3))
 (segment (start 150.1448 105.2195) (end 150.1448 102.135) (width 0.25) (layer B.Cu) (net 3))
 (segment (start 150.1448 102.135) (end 150.1178 102.108) (width 0.25) (layer B.Cu) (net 3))
 (segment (start 200.640699 101.694999) (end 195.6562 96.7105) (width 0.25) (layer B.Cu) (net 4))
 (segment (start 195.6562 96.7105) (end 190.2333 96.7105) (width 0.25) (layer B.Cu) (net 4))
 (segment (start 205.74 102.87) (end 204.564999 101.694999) (width 0.25) (layer B.Cu) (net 4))
 (segment (start 204.564999 101.694999) (end 200.640699 101.694999) (width 0.25) (layer B.Cu) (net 4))
 (segment (start 187.6044 100.3554) (end 188.216701 99.743099) (width 0.25) (layer B.Cu) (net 4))
 (segment (start 188.216701 99.743099) (end 188.216701 98.727099) (width 0.25) (layer B.Cu) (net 4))
 (segment (start 188.216701 98.727099) (end 190.2333 96.7105) (width 0.25) (layer B.Cu) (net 4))
 (segment (start 174.371 103.4796) (end 169.045299 98.153899) (width 0.25) (layer B.Cu) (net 4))
 (segment (start 169.045299 98.153899) (end 127.868001 98.153899) (width 0.25) (layer B.Cu) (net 4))
 (segment (start 121.089699 104.932201) (end 120.7897 105.2322) (width 0.25) (layer B.Cu) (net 4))
 (segment (start 127.868001 98.153899) (end 121.089699 104.932201) (width 0.25) (layer B.Cu) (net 4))
 (segment (start 187.002336 100.5332) (end 177.3174 100.5332) (width 0.25) (layer F.Cu) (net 4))
 (segment (start 177.3174 100.5332) (end 174.371 103.4796) (width 0.25) (layer F.Cu) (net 4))
 (via (at 174.371 103.4796) (size 0.6) (drill 0.4) (layers F.Cu B.Cu) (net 4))
 (segment (start 187.6044 100.3554) (end 187.180136 100.3554) (width 0.25) (layer F.Cu) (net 4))
 (segment (start 187.180136 100.3554) (end 187.002336 100.5332) (width 0.25) (layer F.Cu) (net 4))
 (via (at 187.6044 100.3554) (size 0.6) (drill 0.4) (layers F.Cu B.Cu) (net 4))
 (segment (start 120.7897 105.2322) (end 120.7897 104.5047) (width 0.25) (layer F.Cu) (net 4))
 (segment (start 120.7897 104.5047) (end 117.885 101.6) (width 0.25) (layer F.Cu) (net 4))
 (segment (start 117.885 101.6) (end 117.685 101.6) (width 0.25) (layer F.Cu) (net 4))
 (segment (start 120.7897 105.2322) (end 119.6373 106.3846) (width 0.25) (layer F.Cu) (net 4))
 (segment (start 119.6373 106.3846) (end 117.497 106.3846) (width 0.25) (layer F.Cu) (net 4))
 (segment (start 117.1883 105.2195) (end 120.777 105.2195) (width 0.25) (layer B.Cu) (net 4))
 (segment (start 120.777 105.2195) (end 120.7897 105.2322) (width 0.25) (layer B.Cu) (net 4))
 (via (at 120.7897 105.2322) (size 0.6) (drill 0.4) (layers F.Cu B.Cu) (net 4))
 (segment (start 117.1883 105.2195) (end 117.1883 102.2461) (width 0.25) (layer B.Cu) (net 4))
 (segment (start 117.1883 102.2461) (end 117.3645 102.0699) (width 0.25) (layer B.Cu) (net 4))
 (segment (start 117.3645 102.0699) (end 117.3645 99.0727) (width 0.25) (layer B.Cu) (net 4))
 (segment (start 117.3645 99.0727) (end 117.5258 98.9114) (width 0.25) (layer B.Cu) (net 4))
 (segment (start 171.875 101.6) (end 171.875 97.1961) (width 0.25) (layer F.Cu) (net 5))
 (segment (start 171.875 97.1961) (end 171.878 97.1931) (width 0.25) (layer F.Cu) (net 5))
 (segment (start 168.1734 101.901) (end 171.574 101.901) (width 0.25) (layer F.Cu) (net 5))
 (segment (start 171.574 101.901) (end 171.875 101.6) (width 0.25) (layer F.Cu) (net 5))
 (segment (start 164.8841 101.6165) (end 167.8889 101.6165) (width 0.25) (layer F.Cu) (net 5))
 (segment (start 167.8889 101.6165) (end 168.1734 101.901) (width 0.25) (layer F.Cu) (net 5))
 (segment (start 200.145882 95.835882) (end 182.713218 95.835882) (width 0.25) (layer F.Cu) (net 6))
 (segment (start 203.2 97.79) (end 202.1 97.79) (width 0.25) (layer F.Cu) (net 6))
 (segment (start 202.1 97.79) (end 200.145882 95.835882) (width 0.25) (layer F.Cu) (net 6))
 (segment (start 182.713218 95.835882) (end 181.356 97.1931) (width 0.25) (layer F.Cu) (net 6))
 (segment (start 181.356 97.1931) (end 174.578 97.1931) (width 0.25) (layer F.Cu) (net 6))
 (segment (start 187.4266 103.6447) (end 190.246 106.4641) (width 0.25) (layer F.Cu) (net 7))
 (segment (start 190.246 106.4641) (end 200.943819 106.4641) (width 0.25) (layer F.Cu) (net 7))
 (segment (start 200.943819 106.4641) (end 201.997919 105.41) (width 0.25) (layer F.Cu) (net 7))
 (segment (start 201.997919 105.41) (end 203.2 105.41) (width 0.25) (layer F.Cu) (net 7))
 (segment (start 185.6994 101.9175) (end 185.6994 98.3053) (width 0.25) (layer B.Cu) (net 7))
 (segment (start 185.6994 98.3053) (end 183.7309 96.3368) (width 0.25) (layer B.Cu) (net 7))
 (segment (start 183.7309 96.3368) (end 183.7309 96.2368) (width 0.25) (layer B.Cu) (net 7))
 (segment (start 187.4266 103.6447) (end 185.6994 101.9175) (width 0.25) (layer B.Cu) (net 7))
 (via (at 187.4266 103.6447) (size 0.6) (drill 0.4) (layers F.Cu B.Cu) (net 7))
 (segment (start 181.1909 95.9231) (end 183.4172 95.9231) (width 0.25) (layer B.Cu) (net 7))
 (segment (start 183.4172 95.9231) (end 183.7309 96.2368) (width 0.25) (layer B.Cu) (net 7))
 (segment (start 164.8841 98.9165) (end 165.7841 98.9165) (width 0.25) (layer F.Cu) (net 7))
 (segment (start 165.7841 98.9165) (end 168.7775 95.9231) (width 0.25) (layer F.Cu) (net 7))
 (segment (start 168.7775 95.9231) (end 181.1909 95.9231) (width 0.25) (layer F.Cu) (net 7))
 (via (at 181.1909 95.9231) (size 0.6) (drill 0.4) (layers F.Cu B.Cu) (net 7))
 (segment (start 164.8841 98.9165) (end 164.8841 98.8165) (width 0.25) (layer F.Cu) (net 7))
 (segment (start 164.8841 98.8165) (end 162.5622 96.4946) (width 0.25) (layer F.Cu) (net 7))
 (segment (start 162.5622 96.4946) (end 147.447 96.4946) (width 0.25) (layer F.Cu) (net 7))
 (segment (start 147.447 96.4946) (end 134.44 96.4946) (width 0.25) (layer F.Cu) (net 7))
 (segment (start 134.44 96.4946) (end 132.1689 98.7657) (width 0.25) (layer F.Cu) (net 7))
 (segment (start 132.1689 98.7657) (end 132.1689 98.8657) (width 0.25) (layer F.Cu) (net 7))
 (segment (start 150.495 96.5289) (end 147.4813 96.5289) (width 0.25) (layer B.Cu) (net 7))
 (segment (start 147.4813 96.5289) (end 147.447 96.4946) (width 0.25) (layer B.Cu) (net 7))
 (via (at 147.447 96.4946) (size 0.6) (drill 0.4) (layers F.Cu B.Cu) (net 7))
 (segment (start 132.1689 98.7657) (end 129.4152 96.012) (width 0.25) (layer F.Cu) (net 7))
 (segment (start 129.4152 96.012) (end 115.651364 96.012) (width 0.25) (layer F.Cu) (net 7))
 (segment (start 115.651364 96.012) (end 115.2271 96.012) (width 0.25) (layer F.Cu) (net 7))
 (segment (start 115.2271 96.012) (end 117.3264 96.012) (width 0.25) (layer B.Cu) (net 7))
 (segment (start 117.3264 96.012) (end 117.5258 96.2114) (width 0.25) (layer B.Cu) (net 7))
 (segment (start 105.8672 95.9828) (end 115.1979 95.9828) (width 0.25) (layer F.Cu) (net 7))
 (segment (start 115.1979 95.9828) (end 115.2271 96.012) (width 0.25) (layer F.Cu) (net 7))
 (via (at 115.2271 96.012) (size 0.6) (drill 0.4) (layers F.Cu B.Cu) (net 7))
 (segment (start 135.6487 101.6559) (end 132.2591 101.6559) (width 0.25) (layer F.Cu) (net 8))
 (segment (start 132.2591 101.6559) (end 132.1689 101.5657) (width 0.25) (layer F.Cu) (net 8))
 (segment (start 138.855 101.6) (end 135.7046 101.6) (width 0.25) (layer F.Cu) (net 8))
 (segment (start 135.7046 101.6) (end 135.6487 101.6559) (width 0.25) (layer F.Cu) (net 8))
 (segment (start 138.9596 97.663) (end 138.9596 101.4954) (width 0.25) (layer F.Cu) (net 8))
 (segment (start 138.9596 101.4954) (end 138.855 101.6) (width 0.25) (layer F.Cu) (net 8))
 (segment (start 141.6596 97.663) (end 156.7561 97.663) (width 0.25) (layer F.Cu) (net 9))
 (segment (start 156.7561 97.663) (end 162.3314 103.2383) (width 0.25) (layer F.Cu) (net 9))
 (segment (start 162.3314 103.2383) (end 170.697999 103.2383) (width 0.25) (layer F.Cu) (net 9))
 (segment (start 177.31291 98.25169) (end 188.0811 98.25169) (width 0.25) (layer F.Cu) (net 9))
 (segment (start 170.697999 103.2383) (end 170.697999 103.103399) (width 0.25) (layer F.Cu) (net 9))
 (segment (start 170.697999 103.103399) (end 171.022999 102.778399) (width 0.25) (layer F.Cu) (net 9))
 (segment (start 171.022999 102.778399) (end 171.311591 102.778399) (width 0.25) (layer F.Cu) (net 9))
 (segment (start 172.83981 102.72479) (end 177.31291 98.25169) (width 0.25) (layer F.Cu) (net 9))
 (segment (start 188.0811 98.25169) (end 190.046899 96.285891) (width 0.25) (layer F.Cu) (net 9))
 (segment (start 171.311591 102.778399) (end 171.3652 102.72479) (width 0.25) (layer F.Cu) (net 9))
 (segment (start 171.3652 102.72479) (end 172.83981 102.72479) (width 0.25) (layer F.Cu) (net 9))
 (segment (start 190.046899 96.285891) (end 199.155891 96.285891) (width 0.25) (layer F.Cu) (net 9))
 (segment (start 199.155891 96.285891) (end 203.2 100.33) (width 0.25) (layer F.Cu) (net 9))
 (segment (start 105.8672 98.6828) (end 109.3885 98.6828) (width 0.25) (layer F.Cu) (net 10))
 (segment (start 109.3885 98.6828) (end 109.7242 98.3471) (width 0.25) (layer F.Cu) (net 10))
 (segment (start 109.7242 98.3471) (end 109.7242 97.4471) (width 0.25) (layer F.Cu) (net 10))
 (segment (start 105.9523 104.8258) (end 105.9523 101.7173) (width 0.25) (layer F.Cu) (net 10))
 (segment (start 105.9523 101.7173) (end 105.835 101.6) (width 0.25) (layer F.Cu) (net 10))
 (segment (start 105.835 101.6) (end 105.835 98.715) (width 0.25) (layer F.Cu) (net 10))
 (segment (start 105.835 98.715) (end 105.8672 98.6828) (width 0.25) (layer F.Cu) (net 10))
 (segment (start 171.323 103.4034) (end 171.5516 103.1748) (width 0.25) (layer F.Cu) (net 11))
 (segment (start 171.5516 103.1748) (end 173.02621 103.1748) (width 0.25) (layer F.Cu) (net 11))
 (segment (start 173.02621 103.1748) (end 177.49931 98.7017) (width 0.25) (layer F.Cu) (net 11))
 (segment (start 201.7903 102.87) (end 203.2 102.87) (width 0.25) (layer F.Cu) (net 11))
 (segment (start 177.49931 98.7017) (end 188.267501 98.7017) (width 0.25) (layer F.Cu) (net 11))
 (segment (start 188.267501 98.7017) (end 190.2333 96.7359) (width 0.25) (layer F.Cu) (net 11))
 (segment (start 190.2333 96.7359) (end 195.6562 96.7359) (width 0.25) (layer F.Cu) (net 11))
 (segment (start 195.6562 96.7359) (end 201.7903 102.87) (width 0.25) (layer F.Cu) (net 11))
 (segment (start 171.323 103.4034) (end 167.0431 99.1235) (width 0.25) (layer B.Cu) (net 11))
 (segment (start 167.0431 99.1235) (end 166.961701 99.1235) (width 0.25) (layer B.Cu) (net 11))
 (via (at 171.323 103.4034) (size 0.6) (drill 0.4) (layers F.Cu B.Cu) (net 11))
 (segment (start 124.972499 103.280899) (end 119.1387 97.4471) (width 0.25) (layer F.Cu) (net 11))
 (segment (start 119.1387 97.4471) (end 112.4242 97.4471) (width 0.25) (layer F.Cu) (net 11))
 (segment (start 144.54421 99.58789) (end 140.851201 103.280899) (width 0.25) (layer F.Cu) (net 11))
 (segment (start 140.851201 103.280899) (end 124.972499 103.280899) (width 0.25) (layer F.Cu) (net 11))
 (segment (start 155.3464 99.1235) (end 154.88201 99.58789) (width 0.25) (layer F.Cu) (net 11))
 (segment (start 154.88201 99.58789) (end 144.54421 99.58789) (width 0.25) (layer F.Cu) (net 11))
 (segment (start 166.961701 99.1235) (end 155.3464 99.1235) (width 0.25) (layer B.Cu) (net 11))
 (via (at 155.3464 99.1235) (size 0.6) (drill 0.4) (layers F.Cu B.Cu) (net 11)))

